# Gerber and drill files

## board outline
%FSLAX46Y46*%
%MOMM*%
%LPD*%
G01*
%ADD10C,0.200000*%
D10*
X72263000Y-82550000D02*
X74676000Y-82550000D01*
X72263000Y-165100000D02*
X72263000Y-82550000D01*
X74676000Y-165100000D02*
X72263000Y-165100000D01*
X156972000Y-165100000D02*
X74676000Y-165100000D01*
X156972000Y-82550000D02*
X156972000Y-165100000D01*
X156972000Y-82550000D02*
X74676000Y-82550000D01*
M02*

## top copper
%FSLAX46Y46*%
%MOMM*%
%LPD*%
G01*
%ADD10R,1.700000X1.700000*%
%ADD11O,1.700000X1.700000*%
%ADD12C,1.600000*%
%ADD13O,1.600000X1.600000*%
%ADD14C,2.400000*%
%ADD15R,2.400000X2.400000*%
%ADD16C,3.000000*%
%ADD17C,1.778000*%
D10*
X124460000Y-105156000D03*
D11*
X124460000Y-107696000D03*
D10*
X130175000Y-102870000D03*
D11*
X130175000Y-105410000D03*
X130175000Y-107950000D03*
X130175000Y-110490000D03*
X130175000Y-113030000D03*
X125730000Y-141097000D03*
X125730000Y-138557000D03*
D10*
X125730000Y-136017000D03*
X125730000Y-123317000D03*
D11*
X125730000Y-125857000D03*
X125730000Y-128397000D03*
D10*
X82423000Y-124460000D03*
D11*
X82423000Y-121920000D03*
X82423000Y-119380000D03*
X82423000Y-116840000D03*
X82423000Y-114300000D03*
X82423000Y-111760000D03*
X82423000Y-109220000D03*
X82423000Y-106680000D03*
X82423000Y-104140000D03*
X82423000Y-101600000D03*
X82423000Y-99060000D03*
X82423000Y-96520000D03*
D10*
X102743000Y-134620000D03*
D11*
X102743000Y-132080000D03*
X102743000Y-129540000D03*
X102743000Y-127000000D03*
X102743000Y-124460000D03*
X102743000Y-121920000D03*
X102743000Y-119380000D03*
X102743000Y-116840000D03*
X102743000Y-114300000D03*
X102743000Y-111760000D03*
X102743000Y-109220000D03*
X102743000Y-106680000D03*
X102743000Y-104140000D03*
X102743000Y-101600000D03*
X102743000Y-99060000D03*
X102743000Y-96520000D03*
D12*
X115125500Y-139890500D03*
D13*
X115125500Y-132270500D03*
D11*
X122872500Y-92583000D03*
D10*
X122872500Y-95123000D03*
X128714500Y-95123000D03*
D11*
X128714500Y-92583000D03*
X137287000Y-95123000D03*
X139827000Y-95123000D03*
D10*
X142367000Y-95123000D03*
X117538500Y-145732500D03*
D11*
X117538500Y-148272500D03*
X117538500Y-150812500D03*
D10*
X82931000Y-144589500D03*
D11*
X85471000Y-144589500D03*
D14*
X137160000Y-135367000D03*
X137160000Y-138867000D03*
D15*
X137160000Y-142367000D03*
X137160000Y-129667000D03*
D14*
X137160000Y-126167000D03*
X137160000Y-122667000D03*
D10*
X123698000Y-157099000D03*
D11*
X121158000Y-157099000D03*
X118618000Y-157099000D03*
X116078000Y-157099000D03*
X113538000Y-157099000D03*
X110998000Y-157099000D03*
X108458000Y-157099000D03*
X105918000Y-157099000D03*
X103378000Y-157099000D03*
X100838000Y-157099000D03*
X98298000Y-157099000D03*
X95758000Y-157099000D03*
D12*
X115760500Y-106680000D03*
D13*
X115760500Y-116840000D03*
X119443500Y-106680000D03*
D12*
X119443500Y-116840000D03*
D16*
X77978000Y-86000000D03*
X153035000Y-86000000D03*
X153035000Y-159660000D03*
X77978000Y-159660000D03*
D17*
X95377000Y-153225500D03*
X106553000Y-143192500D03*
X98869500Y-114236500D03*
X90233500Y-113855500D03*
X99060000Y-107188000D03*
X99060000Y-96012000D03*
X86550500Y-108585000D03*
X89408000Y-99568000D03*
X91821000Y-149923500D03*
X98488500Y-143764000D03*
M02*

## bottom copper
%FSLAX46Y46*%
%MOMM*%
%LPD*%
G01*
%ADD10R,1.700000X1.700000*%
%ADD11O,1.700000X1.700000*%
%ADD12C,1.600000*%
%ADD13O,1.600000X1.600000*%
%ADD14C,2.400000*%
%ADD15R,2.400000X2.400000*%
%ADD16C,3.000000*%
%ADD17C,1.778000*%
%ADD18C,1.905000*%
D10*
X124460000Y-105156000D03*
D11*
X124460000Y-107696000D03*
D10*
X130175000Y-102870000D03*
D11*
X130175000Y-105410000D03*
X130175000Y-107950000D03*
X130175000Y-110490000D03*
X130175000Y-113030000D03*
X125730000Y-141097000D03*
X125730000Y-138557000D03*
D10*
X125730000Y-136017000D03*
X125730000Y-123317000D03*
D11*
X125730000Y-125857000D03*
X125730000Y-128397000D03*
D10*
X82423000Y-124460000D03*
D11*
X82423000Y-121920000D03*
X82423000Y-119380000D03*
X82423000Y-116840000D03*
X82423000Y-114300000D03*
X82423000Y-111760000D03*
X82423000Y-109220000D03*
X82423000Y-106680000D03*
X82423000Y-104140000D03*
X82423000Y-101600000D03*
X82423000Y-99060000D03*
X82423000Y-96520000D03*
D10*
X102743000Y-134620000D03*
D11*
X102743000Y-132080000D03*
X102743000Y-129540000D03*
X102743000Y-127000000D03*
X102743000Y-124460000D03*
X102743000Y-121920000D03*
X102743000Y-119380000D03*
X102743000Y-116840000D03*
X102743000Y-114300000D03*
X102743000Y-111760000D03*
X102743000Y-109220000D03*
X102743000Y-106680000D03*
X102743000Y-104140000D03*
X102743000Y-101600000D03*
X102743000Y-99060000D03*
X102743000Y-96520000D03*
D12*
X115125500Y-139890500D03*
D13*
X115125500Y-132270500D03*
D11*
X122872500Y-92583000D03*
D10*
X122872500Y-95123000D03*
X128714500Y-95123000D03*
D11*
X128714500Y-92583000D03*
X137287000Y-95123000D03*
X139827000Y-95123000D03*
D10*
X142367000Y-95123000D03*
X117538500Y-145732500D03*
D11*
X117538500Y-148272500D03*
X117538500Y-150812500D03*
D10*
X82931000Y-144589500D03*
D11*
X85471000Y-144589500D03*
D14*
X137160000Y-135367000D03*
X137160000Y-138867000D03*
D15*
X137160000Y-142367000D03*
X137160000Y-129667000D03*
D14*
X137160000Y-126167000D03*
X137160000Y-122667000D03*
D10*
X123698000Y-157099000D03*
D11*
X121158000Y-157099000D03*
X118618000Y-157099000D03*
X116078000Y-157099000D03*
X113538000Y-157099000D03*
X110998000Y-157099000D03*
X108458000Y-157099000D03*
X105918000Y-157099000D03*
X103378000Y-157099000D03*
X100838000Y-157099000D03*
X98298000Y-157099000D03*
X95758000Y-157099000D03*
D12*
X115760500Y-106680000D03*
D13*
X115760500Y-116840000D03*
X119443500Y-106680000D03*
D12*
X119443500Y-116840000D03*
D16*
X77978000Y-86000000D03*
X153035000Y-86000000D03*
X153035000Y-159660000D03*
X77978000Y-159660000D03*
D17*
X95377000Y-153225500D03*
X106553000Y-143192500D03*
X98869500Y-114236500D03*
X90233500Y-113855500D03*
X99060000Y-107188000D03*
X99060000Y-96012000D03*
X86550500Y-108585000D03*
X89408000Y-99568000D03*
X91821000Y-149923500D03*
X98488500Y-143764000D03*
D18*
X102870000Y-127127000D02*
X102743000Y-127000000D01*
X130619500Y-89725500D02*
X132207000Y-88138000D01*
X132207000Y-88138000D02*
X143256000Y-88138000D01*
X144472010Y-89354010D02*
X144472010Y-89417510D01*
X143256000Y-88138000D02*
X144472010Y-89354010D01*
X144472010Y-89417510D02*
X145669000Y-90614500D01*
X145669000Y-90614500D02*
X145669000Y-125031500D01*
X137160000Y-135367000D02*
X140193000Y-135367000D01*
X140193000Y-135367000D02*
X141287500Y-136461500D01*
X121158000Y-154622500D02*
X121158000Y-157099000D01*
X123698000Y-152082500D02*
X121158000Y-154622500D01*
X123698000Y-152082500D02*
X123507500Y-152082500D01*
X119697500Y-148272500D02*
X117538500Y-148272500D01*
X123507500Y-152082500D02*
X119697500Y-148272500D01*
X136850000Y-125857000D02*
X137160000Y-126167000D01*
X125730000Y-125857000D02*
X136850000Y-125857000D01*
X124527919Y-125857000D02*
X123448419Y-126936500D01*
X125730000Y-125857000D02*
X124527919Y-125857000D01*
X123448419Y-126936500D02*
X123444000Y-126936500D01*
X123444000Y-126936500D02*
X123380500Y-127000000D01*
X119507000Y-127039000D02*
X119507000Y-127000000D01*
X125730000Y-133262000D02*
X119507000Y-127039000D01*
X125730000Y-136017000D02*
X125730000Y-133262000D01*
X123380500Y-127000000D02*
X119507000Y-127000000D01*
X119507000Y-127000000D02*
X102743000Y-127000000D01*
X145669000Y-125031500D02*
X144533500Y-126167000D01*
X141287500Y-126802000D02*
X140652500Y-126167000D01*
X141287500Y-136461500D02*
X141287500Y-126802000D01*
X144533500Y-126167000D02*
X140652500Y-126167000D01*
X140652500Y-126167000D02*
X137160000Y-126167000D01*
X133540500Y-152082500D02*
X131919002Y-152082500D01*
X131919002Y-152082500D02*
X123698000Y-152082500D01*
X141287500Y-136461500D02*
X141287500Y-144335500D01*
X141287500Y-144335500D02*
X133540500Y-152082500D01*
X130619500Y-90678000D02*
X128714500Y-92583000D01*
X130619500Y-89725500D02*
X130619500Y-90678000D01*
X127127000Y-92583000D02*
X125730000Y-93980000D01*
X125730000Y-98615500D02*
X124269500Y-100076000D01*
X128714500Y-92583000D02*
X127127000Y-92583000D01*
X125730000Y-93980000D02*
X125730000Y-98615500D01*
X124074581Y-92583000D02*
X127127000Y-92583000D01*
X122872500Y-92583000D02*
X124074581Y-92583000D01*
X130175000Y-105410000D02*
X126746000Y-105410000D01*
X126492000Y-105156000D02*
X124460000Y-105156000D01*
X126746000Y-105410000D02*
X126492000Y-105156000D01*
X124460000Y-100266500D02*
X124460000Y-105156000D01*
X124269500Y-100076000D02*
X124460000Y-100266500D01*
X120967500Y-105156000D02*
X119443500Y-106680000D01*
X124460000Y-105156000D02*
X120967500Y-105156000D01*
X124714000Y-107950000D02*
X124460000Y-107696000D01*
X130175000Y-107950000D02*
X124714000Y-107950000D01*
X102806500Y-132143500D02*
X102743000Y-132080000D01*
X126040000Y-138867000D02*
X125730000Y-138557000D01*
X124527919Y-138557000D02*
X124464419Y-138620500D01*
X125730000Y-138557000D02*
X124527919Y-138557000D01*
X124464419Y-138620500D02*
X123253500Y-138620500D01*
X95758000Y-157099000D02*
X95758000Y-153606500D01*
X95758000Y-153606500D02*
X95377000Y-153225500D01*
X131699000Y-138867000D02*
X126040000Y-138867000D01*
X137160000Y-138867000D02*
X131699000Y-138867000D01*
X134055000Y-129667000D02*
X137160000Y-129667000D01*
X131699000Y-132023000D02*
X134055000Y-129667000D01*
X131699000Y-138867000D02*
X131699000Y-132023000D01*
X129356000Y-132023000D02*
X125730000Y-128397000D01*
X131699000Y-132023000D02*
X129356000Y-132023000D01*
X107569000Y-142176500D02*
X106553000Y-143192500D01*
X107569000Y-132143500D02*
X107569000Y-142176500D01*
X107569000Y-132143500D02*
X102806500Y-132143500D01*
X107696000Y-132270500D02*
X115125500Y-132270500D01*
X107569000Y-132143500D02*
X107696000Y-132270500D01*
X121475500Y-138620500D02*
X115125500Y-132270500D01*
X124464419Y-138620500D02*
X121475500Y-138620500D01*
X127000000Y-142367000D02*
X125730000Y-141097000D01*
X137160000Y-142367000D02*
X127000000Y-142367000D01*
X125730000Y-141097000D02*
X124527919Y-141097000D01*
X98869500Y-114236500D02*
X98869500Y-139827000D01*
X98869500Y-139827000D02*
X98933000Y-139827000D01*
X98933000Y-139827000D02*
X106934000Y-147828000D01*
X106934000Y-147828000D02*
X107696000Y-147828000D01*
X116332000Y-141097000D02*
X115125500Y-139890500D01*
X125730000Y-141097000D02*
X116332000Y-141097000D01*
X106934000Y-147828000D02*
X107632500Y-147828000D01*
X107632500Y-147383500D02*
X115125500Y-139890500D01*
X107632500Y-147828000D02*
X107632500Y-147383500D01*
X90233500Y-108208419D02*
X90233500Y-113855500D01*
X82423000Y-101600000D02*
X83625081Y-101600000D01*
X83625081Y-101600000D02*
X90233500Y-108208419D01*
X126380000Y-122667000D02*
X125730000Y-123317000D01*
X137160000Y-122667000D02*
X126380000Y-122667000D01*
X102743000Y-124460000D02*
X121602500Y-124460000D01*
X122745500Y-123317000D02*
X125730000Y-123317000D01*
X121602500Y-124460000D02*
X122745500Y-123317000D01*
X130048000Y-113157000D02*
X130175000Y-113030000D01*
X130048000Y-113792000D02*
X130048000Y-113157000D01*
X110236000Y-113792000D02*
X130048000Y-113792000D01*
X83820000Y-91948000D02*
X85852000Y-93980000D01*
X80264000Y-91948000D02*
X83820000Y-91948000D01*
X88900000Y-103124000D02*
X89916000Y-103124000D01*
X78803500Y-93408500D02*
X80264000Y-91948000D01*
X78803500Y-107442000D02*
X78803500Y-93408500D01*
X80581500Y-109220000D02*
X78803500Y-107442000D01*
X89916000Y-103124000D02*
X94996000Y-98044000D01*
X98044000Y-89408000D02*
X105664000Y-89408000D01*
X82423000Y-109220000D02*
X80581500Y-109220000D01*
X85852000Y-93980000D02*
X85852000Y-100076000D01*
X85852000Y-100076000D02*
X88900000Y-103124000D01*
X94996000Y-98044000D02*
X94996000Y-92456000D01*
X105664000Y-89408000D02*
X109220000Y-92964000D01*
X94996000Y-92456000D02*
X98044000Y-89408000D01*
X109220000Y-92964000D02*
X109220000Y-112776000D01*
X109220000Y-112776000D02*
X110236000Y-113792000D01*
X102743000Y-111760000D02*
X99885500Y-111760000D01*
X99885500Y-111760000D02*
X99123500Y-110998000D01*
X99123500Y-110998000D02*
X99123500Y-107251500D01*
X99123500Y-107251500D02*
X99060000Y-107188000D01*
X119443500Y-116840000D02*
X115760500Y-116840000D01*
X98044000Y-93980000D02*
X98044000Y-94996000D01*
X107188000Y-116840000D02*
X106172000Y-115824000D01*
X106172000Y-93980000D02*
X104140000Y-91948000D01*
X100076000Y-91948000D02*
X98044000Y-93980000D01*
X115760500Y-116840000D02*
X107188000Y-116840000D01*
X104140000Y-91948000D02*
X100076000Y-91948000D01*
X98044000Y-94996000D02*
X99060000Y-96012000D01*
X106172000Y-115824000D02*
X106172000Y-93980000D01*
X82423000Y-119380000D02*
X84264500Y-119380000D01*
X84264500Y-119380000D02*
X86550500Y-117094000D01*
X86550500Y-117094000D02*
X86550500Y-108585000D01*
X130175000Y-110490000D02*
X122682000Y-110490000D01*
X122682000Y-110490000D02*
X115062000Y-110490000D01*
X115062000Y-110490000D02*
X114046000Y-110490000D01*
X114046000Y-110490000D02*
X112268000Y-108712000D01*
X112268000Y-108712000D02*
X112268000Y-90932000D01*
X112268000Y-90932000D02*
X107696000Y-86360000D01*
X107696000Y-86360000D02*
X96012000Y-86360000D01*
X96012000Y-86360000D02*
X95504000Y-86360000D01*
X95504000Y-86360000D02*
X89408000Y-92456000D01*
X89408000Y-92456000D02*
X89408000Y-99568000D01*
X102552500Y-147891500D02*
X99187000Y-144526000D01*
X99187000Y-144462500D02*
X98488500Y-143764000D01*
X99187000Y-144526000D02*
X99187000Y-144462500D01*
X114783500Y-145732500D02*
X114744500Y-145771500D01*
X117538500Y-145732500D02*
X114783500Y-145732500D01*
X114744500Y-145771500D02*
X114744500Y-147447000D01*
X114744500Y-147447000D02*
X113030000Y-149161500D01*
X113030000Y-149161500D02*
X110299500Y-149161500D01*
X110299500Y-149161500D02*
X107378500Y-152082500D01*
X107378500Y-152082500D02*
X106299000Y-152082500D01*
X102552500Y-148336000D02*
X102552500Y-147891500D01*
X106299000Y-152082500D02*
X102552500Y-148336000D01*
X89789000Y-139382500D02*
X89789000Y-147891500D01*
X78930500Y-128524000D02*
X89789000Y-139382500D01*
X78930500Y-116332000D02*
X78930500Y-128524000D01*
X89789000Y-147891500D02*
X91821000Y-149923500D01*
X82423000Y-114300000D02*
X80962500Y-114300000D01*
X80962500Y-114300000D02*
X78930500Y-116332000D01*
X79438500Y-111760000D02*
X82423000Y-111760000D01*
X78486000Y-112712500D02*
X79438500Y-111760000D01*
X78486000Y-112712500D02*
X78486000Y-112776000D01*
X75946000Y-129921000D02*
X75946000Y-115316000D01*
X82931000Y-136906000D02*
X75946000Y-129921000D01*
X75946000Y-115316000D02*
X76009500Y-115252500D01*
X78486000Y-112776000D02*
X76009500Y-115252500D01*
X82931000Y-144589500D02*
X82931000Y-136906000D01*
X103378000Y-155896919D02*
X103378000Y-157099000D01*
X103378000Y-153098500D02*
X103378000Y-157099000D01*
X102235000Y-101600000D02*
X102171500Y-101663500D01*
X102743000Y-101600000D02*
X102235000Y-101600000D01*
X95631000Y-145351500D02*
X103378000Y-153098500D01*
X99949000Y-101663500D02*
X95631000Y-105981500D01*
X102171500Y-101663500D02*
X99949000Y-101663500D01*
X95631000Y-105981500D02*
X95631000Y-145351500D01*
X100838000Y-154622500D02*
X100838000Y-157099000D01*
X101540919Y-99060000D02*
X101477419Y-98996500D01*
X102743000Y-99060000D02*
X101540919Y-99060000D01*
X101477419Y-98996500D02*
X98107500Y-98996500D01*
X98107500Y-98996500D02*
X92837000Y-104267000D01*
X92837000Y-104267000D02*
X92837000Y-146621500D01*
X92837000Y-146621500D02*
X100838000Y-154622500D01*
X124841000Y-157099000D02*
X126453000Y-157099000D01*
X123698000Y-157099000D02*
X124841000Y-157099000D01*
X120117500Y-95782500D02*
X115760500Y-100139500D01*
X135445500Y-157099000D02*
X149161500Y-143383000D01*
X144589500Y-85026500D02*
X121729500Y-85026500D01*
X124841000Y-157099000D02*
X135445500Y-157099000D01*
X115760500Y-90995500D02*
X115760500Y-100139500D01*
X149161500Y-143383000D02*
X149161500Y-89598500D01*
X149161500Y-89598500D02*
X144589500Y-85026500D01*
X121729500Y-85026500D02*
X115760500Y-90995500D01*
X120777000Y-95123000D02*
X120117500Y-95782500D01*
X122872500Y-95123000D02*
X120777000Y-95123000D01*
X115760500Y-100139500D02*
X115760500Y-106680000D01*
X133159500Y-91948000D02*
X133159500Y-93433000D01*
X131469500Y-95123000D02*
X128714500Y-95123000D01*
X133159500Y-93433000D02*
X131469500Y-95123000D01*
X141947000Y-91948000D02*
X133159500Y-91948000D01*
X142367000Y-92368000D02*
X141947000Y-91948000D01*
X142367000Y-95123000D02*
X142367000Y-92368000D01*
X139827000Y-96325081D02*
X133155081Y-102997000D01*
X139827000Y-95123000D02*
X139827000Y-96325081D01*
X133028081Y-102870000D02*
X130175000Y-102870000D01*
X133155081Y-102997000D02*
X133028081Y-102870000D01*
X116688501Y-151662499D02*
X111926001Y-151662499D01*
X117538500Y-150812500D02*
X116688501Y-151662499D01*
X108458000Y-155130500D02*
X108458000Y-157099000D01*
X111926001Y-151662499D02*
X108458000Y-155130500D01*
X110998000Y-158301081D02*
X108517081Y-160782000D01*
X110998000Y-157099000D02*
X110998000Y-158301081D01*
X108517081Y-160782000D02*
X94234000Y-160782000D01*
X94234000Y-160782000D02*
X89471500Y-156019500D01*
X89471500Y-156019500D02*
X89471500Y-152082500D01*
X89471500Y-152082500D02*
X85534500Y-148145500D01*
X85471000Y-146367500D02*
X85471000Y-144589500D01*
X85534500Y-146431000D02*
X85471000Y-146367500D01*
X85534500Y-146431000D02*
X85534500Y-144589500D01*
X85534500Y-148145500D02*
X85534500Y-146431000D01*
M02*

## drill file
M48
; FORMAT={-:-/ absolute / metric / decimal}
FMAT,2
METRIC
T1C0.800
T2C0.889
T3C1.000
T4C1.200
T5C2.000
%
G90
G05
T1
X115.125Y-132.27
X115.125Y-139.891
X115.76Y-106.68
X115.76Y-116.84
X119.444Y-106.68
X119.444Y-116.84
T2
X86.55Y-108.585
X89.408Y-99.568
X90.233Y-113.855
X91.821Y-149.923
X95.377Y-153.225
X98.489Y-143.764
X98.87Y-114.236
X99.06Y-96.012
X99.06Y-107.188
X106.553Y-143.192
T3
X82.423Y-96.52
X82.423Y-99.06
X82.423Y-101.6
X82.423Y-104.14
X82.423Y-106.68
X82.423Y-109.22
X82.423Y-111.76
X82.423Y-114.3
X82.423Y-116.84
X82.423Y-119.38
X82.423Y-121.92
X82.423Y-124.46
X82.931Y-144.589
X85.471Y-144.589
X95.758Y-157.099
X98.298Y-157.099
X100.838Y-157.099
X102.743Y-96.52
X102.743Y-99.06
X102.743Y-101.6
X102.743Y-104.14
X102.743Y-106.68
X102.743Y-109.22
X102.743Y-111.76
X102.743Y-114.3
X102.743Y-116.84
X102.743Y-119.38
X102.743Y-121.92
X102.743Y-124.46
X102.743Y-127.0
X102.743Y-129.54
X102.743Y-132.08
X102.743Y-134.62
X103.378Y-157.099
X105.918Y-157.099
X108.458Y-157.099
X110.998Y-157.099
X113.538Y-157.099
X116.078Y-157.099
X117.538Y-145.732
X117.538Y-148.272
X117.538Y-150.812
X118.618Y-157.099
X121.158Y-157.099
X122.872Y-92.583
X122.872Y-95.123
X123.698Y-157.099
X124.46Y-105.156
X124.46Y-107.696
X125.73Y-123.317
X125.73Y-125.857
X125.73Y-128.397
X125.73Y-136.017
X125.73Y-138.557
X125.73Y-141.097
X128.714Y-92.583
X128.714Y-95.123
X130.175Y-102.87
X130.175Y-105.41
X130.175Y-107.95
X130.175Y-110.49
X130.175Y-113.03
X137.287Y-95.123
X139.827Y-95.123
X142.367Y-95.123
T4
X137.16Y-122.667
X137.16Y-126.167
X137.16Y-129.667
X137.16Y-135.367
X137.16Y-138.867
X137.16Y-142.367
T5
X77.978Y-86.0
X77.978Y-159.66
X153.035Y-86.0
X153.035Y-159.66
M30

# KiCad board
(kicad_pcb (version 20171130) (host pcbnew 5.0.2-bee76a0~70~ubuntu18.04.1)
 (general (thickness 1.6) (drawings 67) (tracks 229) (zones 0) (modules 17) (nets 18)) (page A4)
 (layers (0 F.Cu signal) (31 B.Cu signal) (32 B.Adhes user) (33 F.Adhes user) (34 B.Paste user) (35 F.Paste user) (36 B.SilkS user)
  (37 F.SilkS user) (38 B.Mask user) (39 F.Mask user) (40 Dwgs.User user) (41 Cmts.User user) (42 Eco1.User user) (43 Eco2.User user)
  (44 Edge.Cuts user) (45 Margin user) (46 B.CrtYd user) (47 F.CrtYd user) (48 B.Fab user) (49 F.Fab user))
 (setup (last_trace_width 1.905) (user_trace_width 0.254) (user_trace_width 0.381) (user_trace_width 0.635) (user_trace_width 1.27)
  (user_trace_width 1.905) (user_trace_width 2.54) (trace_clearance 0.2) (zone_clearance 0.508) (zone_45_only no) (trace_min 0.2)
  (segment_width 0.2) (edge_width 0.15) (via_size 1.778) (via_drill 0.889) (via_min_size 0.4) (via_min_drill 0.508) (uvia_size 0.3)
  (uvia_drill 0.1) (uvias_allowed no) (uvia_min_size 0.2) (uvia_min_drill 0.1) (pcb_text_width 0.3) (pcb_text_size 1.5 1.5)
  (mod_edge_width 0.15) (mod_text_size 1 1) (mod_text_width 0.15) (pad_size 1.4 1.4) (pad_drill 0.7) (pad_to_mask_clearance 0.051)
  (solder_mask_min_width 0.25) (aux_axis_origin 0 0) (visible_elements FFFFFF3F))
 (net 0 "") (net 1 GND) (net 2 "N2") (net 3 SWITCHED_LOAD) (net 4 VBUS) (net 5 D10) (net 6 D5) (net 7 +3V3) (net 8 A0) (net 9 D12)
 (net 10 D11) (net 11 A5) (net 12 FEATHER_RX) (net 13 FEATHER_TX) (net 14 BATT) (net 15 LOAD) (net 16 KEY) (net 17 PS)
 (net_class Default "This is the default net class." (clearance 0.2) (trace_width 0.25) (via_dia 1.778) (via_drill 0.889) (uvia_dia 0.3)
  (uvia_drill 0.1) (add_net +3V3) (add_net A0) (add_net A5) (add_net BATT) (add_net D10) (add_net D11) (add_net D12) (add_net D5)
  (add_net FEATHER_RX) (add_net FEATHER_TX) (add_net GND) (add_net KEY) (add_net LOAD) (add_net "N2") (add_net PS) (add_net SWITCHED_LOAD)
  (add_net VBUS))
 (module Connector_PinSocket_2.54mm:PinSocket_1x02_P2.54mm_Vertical (layer F.Cu) (at 124.46 105.156)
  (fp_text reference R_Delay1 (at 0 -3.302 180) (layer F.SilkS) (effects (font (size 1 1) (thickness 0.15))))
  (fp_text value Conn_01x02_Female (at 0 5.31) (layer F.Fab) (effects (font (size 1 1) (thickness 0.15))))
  (pad 1 thru_hole rect (at 0 0) (size 1.7 1.7) (drill 1) (layers *.Cu *.Mask) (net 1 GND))
  (pad 2 thru_hole oval (at 0 2.54) (size 1.7 1.7) (drill 1) (layers *.Cu *.Mask) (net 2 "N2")))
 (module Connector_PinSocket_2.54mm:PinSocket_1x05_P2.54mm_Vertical (layer F.Cu) (at 130.175 102.87)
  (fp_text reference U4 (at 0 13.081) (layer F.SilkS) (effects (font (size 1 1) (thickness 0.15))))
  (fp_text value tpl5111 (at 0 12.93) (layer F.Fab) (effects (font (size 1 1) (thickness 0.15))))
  (pad 1 thru_hole rect (at 0 0) (size 1.7 1.7) (drill 1) (layers *.Cu *.Mask) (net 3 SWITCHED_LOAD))
  (pad 2 thru_hole oval (at 0 2.54) (size 1.7 1.7) (drill 1) (layers *.Cu *.Mask) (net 1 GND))
  (pad 3 thru_hole oval (at 0 5.08) (size 1.7 1.7) (drill 1) (layers *.Cu *.Mask) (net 2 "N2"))
  (pad 4 thru_hole oval (at 0 7.62) (size 1.7 1.7) (drill 1) (layers *.Cu *.Mask) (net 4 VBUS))
  (pad 5 thru_hole oval (at 0 10.16) (size 1.7 1.7) (drill 1) (layers *.Cu *.Mask) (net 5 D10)))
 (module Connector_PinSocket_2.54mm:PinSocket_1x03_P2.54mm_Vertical (layer F.Cu) (at 125.73 136.017)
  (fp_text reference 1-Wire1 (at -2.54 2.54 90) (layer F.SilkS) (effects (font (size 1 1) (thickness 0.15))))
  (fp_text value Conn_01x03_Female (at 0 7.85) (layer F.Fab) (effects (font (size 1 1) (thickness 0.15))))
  (pad 3 thru_hole oval (at 0 5.08) (size 1.7 1.7) (drill 1) (layers *.Cu *.Mask) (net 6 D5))
  (pad 2 thru_hole oval (at 0 2.54) (size 1.7 1.7) (drill 1) (layers *.Cu *.Mask) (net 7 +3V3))
  (pad 1 thru_hole rect (at 0 0) (size 1.7 1.7) (drill 1) (layers *.Cu *.Mask) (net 1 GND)))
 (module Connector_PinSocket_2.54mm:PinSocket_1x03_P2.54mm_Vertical (layer F.Cu) (at 125.73 123.317)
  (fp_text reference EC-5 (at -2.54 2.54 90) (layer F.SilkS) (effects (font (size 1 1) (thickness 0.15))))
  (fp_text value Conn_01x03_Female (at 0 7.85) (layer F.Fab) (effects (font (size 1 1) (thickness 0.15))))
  (pad 1 thru_hole rect (at 0 0) (size 1.7 1.7) (drill 1) (layers *.Cu *.Mask) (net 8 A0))
  (pad 2 thru_hole oval (at 0 2.54) (size 1.7 1.7) (drill 1) (layers *.Cu *.Mask) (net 1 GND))
  (pad 3 thru_hole oval (at 0 5.08) (size 1.7 1.7) (drill 1) (layers *.Cu *.Mask) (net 7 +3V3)))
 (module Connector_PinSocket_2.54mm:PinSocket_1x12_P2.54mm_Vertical (layer F.Cu) (at 82.423 124.46 180)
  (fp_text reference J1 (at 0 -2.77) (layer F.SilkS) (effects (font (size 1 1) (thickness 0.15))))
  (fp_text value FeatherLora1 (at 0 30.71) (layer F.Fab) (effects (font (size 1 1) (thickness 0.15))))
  (pad 1 thru_hole rect (at 0 0 180) (size 1.7 1.7) (drill 1) (layers *.Cu *.Mask))
  (pad 2 thru_hole oval (at 0 2.54 180) (size 1.7 1.7) (drill 1) (layers *.Cu *.Mask))
  (pad 3 thru_hole oval (at 0 5.08 180) (size 1.7 1.7) (drill 1) (layers *.Cu *.Mask) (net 4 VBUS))
  (pad 4 thru_hole oval (at 0 7.62 180) (size 1.7 1.7) (drill 1) (layers *.Cu *.Mask))
  (pad 5 thru_hole oval (at 0 10.16 180) (size 1.7 1.7) (drill 1) (layers *.Cu *.Mask) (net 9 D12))
  (pad 6 thru_hole oval (at 0 12.7 180) (size 1.7 1.7) (drill 1) (layers *.Cu *.Mask) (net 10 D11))
  (pad 7 thru_hole oval (at 0 15.24 180) (size 1.7 1.7) (drill 1) (layers *.Cu *.Mask) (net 5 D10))
  (pad 8 thru_hole oval (at 0 17.78 180) (size 1.7 1.7) (drill 1) (layers *.Cu *.Mask))
  (pad 9 thru_hole oval (at 0 20.32 180) (size 1.7 1.7) (drill 1) (layers *.Cu *.Mask))
  (pad 10 thru_hole oval (at 0 22.86 180) (size 1.7 1.7) (drill 1) (layers *.Cu *.Mask) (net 6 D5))
  (pad 11 thru_hole oval (at 0 25.4 180) (size 1.7 1.7) (drill 1) (layers *.Cu *.Mask))
  (pad 12 thru_hole oval (at 0 27.94 180) (size 1.7 1.7) (drill 1) (layers *.Cu *.Mask)))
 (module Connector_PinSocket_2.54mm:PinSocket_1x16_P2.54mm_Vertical (layer F.Cu) (at 102.743 134.62 180)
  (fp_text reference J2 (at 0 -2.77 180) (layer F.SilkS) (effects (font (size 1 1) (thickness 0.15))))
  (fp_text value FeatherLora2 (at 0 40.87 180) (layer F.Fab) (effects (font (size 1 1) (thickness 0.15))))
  (pad 1 thru_hole rect (at 0 0 180) (size 1.7 1.7) (drill 1) (layers *.Cu *.Mask))
  (pad 2 thru_hole oval (at 0 2.54 180) (size 1.7 1.7) (drill 1) (layers *.Cu *.Mask) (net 7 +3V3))
  (pad 3 thru_hole oval (at 0 5.08 180) (size 1.7 1.7) (drill 1) (layers *.Cu *.Mask))
  (pad 4 thru_hole oval (at 0 7.62 180) (size 1.7 1.7) (drill 1) (layers *.Cu *.Mask) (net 1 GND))
  (pad 5 thru_hole oval (at 0 10.16 180) (size 1.7 1.7) (drill 1) (layers *.Cu *.Mask) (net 8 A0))
  (pad 6 thru_hole oval (at 0 12.7 180) (size 1.7 1.7) (drill 1) (layers *.Cu *.Mask))
  (pad 7 thru_hole oval (at 0 15.24 180) (size 1.7 1.7) (drill 1) (layers *.Cu *.Mask))
  (pad 8 thru_hole oval (at 0 17.78 180) (size 1.7 1.7) (drill 1) (layers *.Cu *.Mask))
  (pad 9 thru_hole oval (at 0 20.32 180) (size 1.7 1.7) (drill 1) (layers *.Cu *.Mask))
  (pad 10 thru_hole oval (at 0 22.86 180) (size 1.7 1.7) (drill 1) (layers *.Cu *.Mask) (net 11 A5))
  (pad 11 thru_hole oval (at 0 25.4 180) (size 1.7 1.7) (drill 1) (layers *.Cu *.Mask))
  (pad 12 thru_hole oval (at 0 27.94 180) (size 1.7 1.7) (drill 1) (layers *.Cu *.Mask))
  (pad 13 thru_hole oval (at 0 30.48 180) (size 1.7 1.7) (drill 1) (layers *.Cu *.Mask))
  (pad 14 thru_hole oval (at 0 33.02 180) (size 1.7 1.7) (drill 1) (layers *.Cu *.Mask) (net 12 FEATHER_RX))
  (pad 15 thru_hole oval (at 0 35.56 180) (size 1.7 1.7) (drill 1) (layers *.Cu *.Mask) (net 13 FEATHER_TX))
  (pad 16 thru_hole oval (at 0 38.1 180) (size 1.7 1.7) (drill 1) (layers *.Cu *.Mask)))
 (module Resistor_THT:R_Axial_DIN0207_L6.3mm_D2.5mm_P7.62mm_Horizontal (layer F.Cu) (at 115.1255 139.8905 90)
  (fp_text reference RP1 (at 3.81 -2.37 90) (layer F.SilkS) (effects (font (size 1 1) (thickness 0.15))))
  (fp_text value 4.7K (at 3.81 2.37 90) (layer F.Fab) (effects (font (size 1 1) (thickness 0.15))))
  (pad 1 thru_hole circle (at 0 0 90) (size 1.6 1.6) (drill 0.8) (layers *.Cu *.Mask) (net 6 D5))
  (pad 2 thru_hole oval (at 7.62 0 90) (size 1.6 1.6) (drill 0.8) (layers *.Cu *.Mask) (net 7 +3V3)))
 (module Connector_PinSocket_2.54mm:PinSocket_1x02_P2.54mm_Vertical (layer F.Cu) (at 122.8725 95.123 180)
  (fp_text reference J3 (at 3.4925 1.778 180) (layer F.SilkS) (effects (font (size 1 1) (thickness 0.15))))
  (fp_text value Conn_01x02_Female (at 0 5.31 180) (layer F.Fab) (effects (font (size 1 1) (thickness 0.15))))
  (pad 2 thru_hole oval (at 0 2.54 180) (size 1.7 1.7) (drill 1) (layers *.Cu *.Mask) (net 1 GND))
  (pad 1 thru_hole rect (at 0 0 180) (size 1.7 1.7) (drill 1) (layers *.Cu *.Mask) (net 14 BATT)))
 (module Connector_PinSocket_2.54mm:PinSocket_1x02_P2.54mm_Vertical (layer F.Cu) (at 128.7145 95.123 180)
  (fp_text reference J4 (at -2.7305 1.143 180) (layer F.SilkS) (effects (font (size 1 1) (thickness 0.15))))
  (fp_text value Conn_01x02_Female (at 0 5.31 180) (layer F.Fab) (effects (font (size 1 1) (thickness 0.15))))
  (pad 1 thru_hole rect (at 0 0 180) (size 1.7 1.7) (drill 1) (layers *.Cu *.Mask) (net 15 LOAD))
  (pad 2 thru_hole oval (at 0 2.54 180) (size 1.7 1.7) (drill 1) (layers *.Cu *.Mask) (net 1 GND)))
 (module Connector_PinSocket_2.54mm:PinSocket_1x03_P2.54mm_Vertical (layer F.Cu) (at 142.367 95.123 270)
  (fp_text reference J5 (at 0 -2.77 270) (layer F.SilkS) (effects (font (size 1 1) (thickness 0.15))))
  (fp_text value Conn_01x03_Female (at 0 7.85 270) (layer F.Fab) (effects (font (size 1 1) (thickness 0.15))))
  (pad 3 thru_hole oval (at 0 5.08 270) (size 1.7 1.7) (drill 1) (layers *.Cu *.Mask))
  (pad 2 thru_hole oval (at 0 2.54 270) (size 1.7 1.7) (drill 1) (layers *.Cu *.Mask) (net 3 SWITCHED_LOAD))
  (pad 1 thru_hole rect (at 0 0 270) (size 1.7 1.7) (drill 1) (layers *.Cu *.Mask) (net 15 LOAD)))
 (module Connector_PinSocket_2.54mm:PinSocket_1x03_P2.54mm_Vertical (layer F.Cu) (at 117.5385 145.7325)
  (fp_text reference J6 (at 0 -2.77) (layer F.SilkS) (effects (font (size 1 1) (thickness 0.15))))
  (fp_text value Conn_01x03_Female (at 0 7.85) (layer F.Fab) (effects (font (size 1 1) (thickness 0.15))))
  (pad 1 thru_hole rect (at 0 0) (size 1.7 1.7) (drill 1) (layers *.Cu *.Mask) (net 9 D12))
  (pad 2 thru_hole oval (at 0 2.54) (size 1.7 1.7) (drill 1) (layers *.Cu *.Mask) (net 1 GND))
  (pad 3 thru_hole oval (at 0 5.08) (size 1.7 1.7) (drill 1) (layers *.Cu *.Mask) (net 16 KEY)))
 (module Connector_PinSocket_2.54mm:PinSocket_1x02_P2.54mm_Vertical (layer F.Cu) (at 82.931 144.5895 90)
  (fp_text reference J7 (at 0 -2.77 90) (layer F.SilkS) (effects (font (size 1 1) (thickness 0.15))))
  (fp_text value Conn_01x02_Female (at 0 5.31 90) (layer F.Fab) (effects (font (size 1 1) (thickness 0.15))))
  (pad 1 thru_hole rect (at 0 0 90) (size 1.7 1.7) (drill 1) (layers *.Cu *.Mask) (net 10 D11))
  (pad 2 thru_hole oval (at 0 2.54 90) (size 1.7 1.7) (drill 1) (layers *.Cu *.Mask) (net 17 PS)))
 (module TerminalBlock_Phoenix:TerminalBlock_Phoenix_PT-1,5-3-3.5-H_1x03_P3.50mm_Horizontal (layer F.Cu) (at 137.16 142.367 90)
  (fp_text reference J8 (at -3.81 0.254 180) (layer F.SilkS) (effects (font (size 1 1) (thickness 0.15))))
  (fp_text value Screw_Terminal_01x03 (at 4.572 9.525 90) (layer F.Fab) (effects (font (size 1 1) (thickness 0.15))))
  (pad 3 thru_hole circle (at 7 0 90) (size 2.4 2.4) (drill 1.2) (layers *.Cu *.Mask) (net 1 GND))
  (pad 2 thru_hole circle (at 3.5 0 90) (size 2.4 2.4) (drill 1.2) (layers *.Cu *.Mask) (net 7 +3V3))
  (pad 1 thru_hole rect (at 0 0 90) (size 2.4 2.4) (drill 1.2) (layers *.Cu *.Mask) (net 6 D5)))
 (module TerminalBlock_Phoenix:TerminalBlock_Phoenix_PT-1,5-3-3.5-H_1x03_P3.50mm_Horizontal (layer F.Cu) (at 137.16 129.667 90)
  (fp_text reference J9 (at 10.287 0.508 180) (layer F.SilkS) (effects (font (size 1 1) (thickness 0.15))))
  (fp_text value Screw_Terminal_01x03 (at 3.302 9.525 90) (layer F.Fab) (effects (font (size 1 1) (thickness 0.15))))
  (pad 1 thru_hole rect (at 0 0 90) (size 2.4 2.4) (drill 1.2) (layers *.Cu *.Mask) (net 7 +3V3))
  (pad 2 thru_hole circle (at 3.5 0 90) (size 2.4 2.4) (drill 1.2) (layers *.Cu *.Mask) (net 1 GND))
  (pad 3 thru_hole circle (at 7 0 90) (size 2.4 2.4) (drill 1.2) (layers *.Cu *.Mask) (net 8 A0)))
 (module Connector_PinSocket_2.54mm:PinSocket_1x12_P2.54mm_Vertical (layer F.Cu) (at 123.698 157.099 270)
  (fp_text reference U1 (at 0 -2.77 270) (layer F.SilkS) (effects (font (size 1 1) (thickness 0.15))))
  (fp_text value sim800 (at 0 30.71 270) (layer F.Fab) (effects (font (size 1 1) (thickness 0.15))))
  (pad 1 thru_hole rect (at 0 0 270) (size 1.7 1.7) (drill 1) (layers *.Cu *.Mask) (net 14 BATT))
  (pad 2 thru_hole oval (at 0 2.54 270) (size 1.7 1.7) (drill 1) (layers *.Cu *.Mask) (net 1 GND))
  (pad 3 thru_hole oval (at 0 5.08 270) (size 1.7 1.7) (drill 1) (layers *.Cu *.Mask))
  (pad 4 thru_hole oval (at 0 7.62 270) (size 1.7 1.7) (drill 1) (layers *.Cu *.Mask))
  (pad 5 thru_hole oval (at 0 10.16 270) (size 1.7 1.7) (drill 1) (layers *.Cu *.Mask))
  (pad 6 thru_hole oval (at 0 12.7 270) (size 1.7 1.7) (drill 1) (layers *.Cu *.Mask) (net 17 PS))
  (pad 7 thru_hole oval (at 0 15.24 270) (size 1.7 1.7) (drill 1) (layers *.Cu *.Mask) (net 16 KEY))
  (pad 8 thru_hole oval (at 0 17.78 270) (size 1.7 1.7) (drill 1) (layers *.Cu *.Mask))
  (pad 9 thru_hole oval (at 0 20.32 270) (size 1.7 1.7) (drill 1) (layers *.Cu *.Mask) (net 12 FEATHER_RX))
  (pad 10 thru_hole oval (at 0 22.86 270) (size 1.7 1.7) (drill 1) (layers *.Cu *.Mask) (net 13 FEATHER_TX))
  (pad 11 thru_hole oval (at 0 25.4 270) (size 1.7 1.7) (drill 1) (layers *.Cu *.Mask))
  (pad 12 thru_hole oval (at 0 27.94 270) (size 1.7 1.7) (drill 1) (layers *.Cu *.Mask) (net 7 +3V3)))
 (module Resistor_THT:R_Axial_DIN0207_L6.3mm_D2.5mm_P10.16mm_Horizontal (layer F.Cu) (at 115.7605 106.68 270)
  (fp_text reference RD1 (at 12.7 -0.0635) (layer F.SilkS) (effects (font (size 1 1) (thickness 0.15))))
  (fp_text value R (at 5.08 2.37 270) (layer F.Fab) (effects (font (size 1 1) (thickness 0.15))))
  (pad 1 thru_hole circle (at 0 0 270) (size 1.6 1.6) (drill 0.8) (layers *.Cu *.Mask) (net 14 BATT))
  (pad 2 thru_hole oval (at 10.16 0 270) (size 1.6 1.6) (drill 0.8) (layers *.Cu *.Mask) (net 11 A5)))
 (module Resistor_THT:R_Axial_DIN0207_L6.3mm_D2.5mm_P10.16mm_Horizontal (layer F.Cu) (at 119.4435 116.84 90)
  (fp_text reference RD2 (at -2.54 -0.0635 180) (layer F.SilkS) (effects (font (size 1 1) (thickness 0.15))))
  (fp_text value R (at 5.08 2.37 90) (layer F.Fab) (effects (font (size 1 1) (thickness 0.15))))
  (pad 2 thru_hole oval (at 10.16 0 90) (size 1.6 1.6) (drill 0.8) (layers *.Cu *.Mask) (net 1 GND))
  (pad 1 thru_hole circle (at 0 0 90) (size 1.6 1.6) (drill 0.8) (layers *.Cu *.Mask) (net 11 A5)))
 (gr_line (start 72.263 82.55) (end 74.676 82.55) (layer Edge.Cuts) (width 0.2))
 (gr_line (start 72.263 165.1) (end 72.263 82.55) (layer Edge.Cuts) (width 0.2))
 (gr_line (start 74.676 165.1) (end 72.263 165.1) (layer Edge.Cuts) (width 0.2))
 (gr_line (start 156.972 165.1) (end 74.676 165.1) (layer Edge.Cuts) (width 0.2))
 (gr_line (start 156.972 82.55) (end 156.972 165.1) (layer Edge.Cuts) (width 0.2))
 (gr_line (start 156.972 82.55) (end 74.676 82.55) (layer Edge.Cuts) (width 0.2))
 (via (at 77.978 86) (size 3) (drill 2) (layers F.Cu B.Cu) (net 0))
 (via (at 153.035 86) (size 3) (drill 2) (layers F.Cu B.Cu) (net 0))
 (via (at 153.035 159.66) (size 3) (drill 2) (layers F.Cu B.Cu) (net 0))
 (via (at 77.978 159.66) (size 3) (drill 2) (layers F.Cu B.Cu) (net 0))
 (segment (start 102.87 127.127) (end 102.743 127) (width 1.905) (layer B.Cu) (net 1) (status 30))
 (segment (start 130.6195 89.7255) (end 132.207 88.138) (width 1.905) (layer B.Cu) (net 1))
 (segment (start 132.207 88.138) (end 143.256 88.138) (width 1.905) (layer B.Cu) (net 1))
 (segment (start 144.47201 89.35401) (end 144.47201 89.41751) (width 1.905) (layer B.Cu) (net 1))
 (segment (start 143.256 88.138) (end 144.47201 89.35401) (width 1.905) (layer B.Cu) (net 1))
 (segment (start 144.47201 89.41751) (end 145.669 90.6145) (width 1.905) (layer B.Cu) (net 1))
 (segment (start 145.669 90.6145) (end 145.669 125.0315) (width 1.905) (layer B.Cu) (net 1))
 (segment (start 137.16 135.367) (end 140.193 135.367) (width 1.905) (layer B.Cu) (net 1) (status 10))
 (segment (start 140.193 135.367) (end 141.2875 136.4615) (width 1.905) (layer B.Cu) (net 1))
 (segment (start 121.158 154.6225) (end 121.158 157.099) (width 1.905) (layer B.Cu) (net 1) (status 20))
 (segment (start 123.698 152.0825) (end 121.158 154.6225) (width 1.905) (layer B.Cu) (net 1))
 (segment (start 123.698 152.0825) (end 123.5075 152.0825) (width 1.905) (layer B.Cu) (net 1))
 (segment (start 119.6975 148.2725) (end 117.5385 148.2725) (width 1.905) (layer B.Cu) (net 1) (status 20))
 (segment (start 123.5075 152.0825) (end 119.6975 148.2725) (width 1.905) (layer B.Cu) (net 1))
 (segment (start 136.85 125.857) (end 137.16 126.167) (width 1.905) (layer B.Cu) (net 1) (status 30))
 (segment (start 125.73 125.857) (end 136.85 125.857) (width 1.905) (layer B.Cu) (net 1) (status 30))
 (segment (start 124.527919 125.857) (end 123.448419 126.9365) (width 1.905) (layer B.Cu) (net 1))
 (segment (start 125.73 125.857) (end 124.527919 125.857) (width 1.905) (layer B.Cu) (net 1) (status 10))
 (segment (start 123.448419 126.9365) (end 123.444 126.9365) (width 1.905) (layer B.Cu) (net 1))
 (segment (start 123.444 126.9365) (end 123.3805 127) (width 1.905) (layer B.Cu) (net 1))
 (segment (start 119.507 127.039) (end 119.507 127) (width 1.905) (layer B.Cu) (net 1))
 (segment (start 125.73 133.262) (end 119.507 127.039) (width 1.905) (layer B.Cu) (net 1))
 (segment (start 125.73 136.017) (end 125.73 133.262) (width 1.905) (layer B.Cu) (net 1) (status 10))
 (segment (start 123.3805 127) (end 119.507 127) (width 1.905) (layer B.Cu) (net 1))
 (segment (start 119.507 127) (end 102.743 127) (width 1.905) (layer B.Cu) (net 1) (status 20))
 (segment (start 145.669 125.0315) (end 144.5335 126.167) (width 1.905) (layer B.Cu) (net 1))
 (segment (start 141.2875 126.802) (end 140.6525 126.167) (width 1.905) (layer B.Cu) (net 1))
 (segment (start 141.2875 136.4615) (end 141.2875 126.802) (width 1.905) (layer B.Cu) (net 1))
 (segment (start 144.5335 126.167) (end 140.6525 126.167) (width 1.905) (layer B.Cu) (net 1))
 (segment (start 140.6525 126.167) (end 137.16 126.167) (width 1.905) (layer B.Cu) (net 1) (status 20))
 (segment (start 133.5405 152.0825) (end 131.919002 152.0825) (width 1.905) (layer B.Cu) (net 1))
 (segment (start 131.919002 152.0825) (end 123.698 152.0825) (width 1.905) (layer B.Cu) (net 1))
 (segment (start 141.2875 136.4615) (end 141.2875 144.3355) (width 1.905) (layer B.Cu) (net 1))
 (segment (start 141.2875 144.3355) (end 133.5405 152.0825) (width 1.905) (layer B.Cu) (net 1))
 (segment (start 130.6195 90.678) (end 128.7145 92.583) (width 1.905) (layer B.Cu) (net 1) (status 20))
 (segment (start 130.6195 89.7255) (end 130.6195 90.678) (width 1.905) (layer B.Cu) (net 1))
 (segment (start 127.127 92.583) (end 125.73 93.98) (width 1.905) (layer B.Cu) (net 1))
 (segment (start 125.73 98.6155) (end 124.2695 100.076) (width 1.905) (layer B.Cu) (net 1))
 (segment (start 128.7145 92.583) (end 127.127 92.583) (width 1.905) (layer B.Cu) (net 1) (status 10))
 (segment (start 125.73 93.98) (end 125.73 98.6155) (width 1.905) (layer B.Cu) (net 1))
 (segment (start 124.074581 92.583) (end 127.127 92.583) (width 1.905) (layer B.Cu) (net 1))
 (segment (start 122.8725 92.583) (end 124.074581 92.583) (width 1.905) (layer B.Cu) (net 1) (status 10))
 (segment (start 130.175 105.41) (end 126.746 105.41) (width 1.905) (layer B.Cu) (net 1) (status 10))
 (segment (start 126.492 105.156) (end 124.46 105.156) (width 1.905) (layer B.Cu) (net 1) (status 20))
 (segment (start 126.746 105.41) (end 126.492 105.156) (width 1.905) (layer B.Cu) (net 1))
 (segment (start 124.46 100.2665) (end 124.46 105.156) (width 1.905) (layer B.Cu) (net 1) (status 20))
 (segment (start 124.2695 100.076) (end 124.46 100.2665) (width 1.905) (layer B.Cu) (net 1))
 (segment (start 120.9675 105.156) (end 119.4435 106.68) (width 1.905) (layer B.Cu) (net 1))
 (segment (start 124.46 105.156) (end 120.9675 105.156) (width 1.905) (layer B.Cu) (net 1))
 (segment (start 124.714 107.95) (end 124.46 107.696) (width 1.905) (layer B.Cu) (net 2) (status 30))
 (segment (start 130.175 107.95) (end 124.714 107.95) (width 1.905) (layer B.Cu) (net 2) (status 30))
 (segment (start 102.8065 132.1435) (end 102.743 132.08) (width 1.905) (layer B.Cu) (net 7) (status 30))
 (segment (start 126.04 138.867) (end 125.73 138.557) (width 1.905) (layer B.Cu) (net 7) (status 30))
 (segment (start 124.527919 138.557) (end 124.464419 138.6205) (width 1.905) (layer B.Cu) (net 7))
 (segment (start 125.73 138.557) (end 124.527919 138.557) (width 1.905) (layer B.Cu) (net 7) (status 10))
 (segment (start 124.464419 138.6205) (end 123.2535 138.6205) (width 1.905) (layer B.Cu) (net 7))
 (segment (start 95.758 157.099) (end 95.758 153.6065) (width 1.905) (layer B.Cu) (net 7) (status 10))
 (via (at 95.377 153.2255) (size 1.778) (drill 0.889) (layers F.Cu B.Cu) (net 7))
 (segment (start 95.758 153.6065) (end 95.377 153.2255) (width 1.905) (layer B.Cu) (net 7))
 (segment (start 131.699 138.867) (end 126.04 138.867) (width 1.905) (layer B.Cu) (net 7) (status 20))
 (segment (start 137.16 138.867) (end 131.699 138.867) (width 1.905) (layer B.Cu) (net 7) (status 10))
 (segment (start 134.055 129.667) (end 137.16 129.667) (width 1.905) (layer B.Cu) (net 7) (status 20))
 (segment (start 131.699 132.023) (end 134.055 129.667) (width 1.905) (layer B.Cu) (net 7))
 (segment (start 131.699 138.867) (end 131.699 132.023) (width 1.905) (layer B.Cu) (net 7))
 (segment (start 129.356 132.023) (end 125.73 128.397) (width 1.905) (layer B.Cu) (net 7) (status 20))
 (segment (start 131.699 132.023) (end 129.356 132.023) (width 1.905) (layer B.Cu) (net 7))
 (via (at 106.553 143.1925) (size 1.778) (drill 0.889) (layers F.Cu B.Cu) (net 7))
 (segment (start 107.569 142.1765) (end 106.553 143.1925) (width 1.905) (layer B.Cu) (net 7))
 (segment (start 107.569 132.1435) (end 107.569 142.1765) (width 1.905) (layer B.Cu) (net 7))
 (segment (start 107.569 132.1435) (end 102.8065 132.1435) (width 1.905) (layer B.Cu) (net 7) (status 20))
 (segment (start 107.696 132.2705) (end 115.1255 132.2705) (width 1.905) (layer B.Cu) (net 7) (status 20))
 (segment (start 107.569 132.1435) (end 107.696 132.2705) (width 1.905) (layer B.Cu) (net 7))
 (segment (start 121.4755 138.6205) (end 115.1255 132.2705) (width 1.905) (layer B.Cu) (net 7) (status 20))
 (segment (start 124.464419 138.6205) (end 121.4755 138.6205) (width 1.905) (layer B.Cu) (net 7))
 (via (at 98.8695 114.2365) (size 1.778) (drill 0.889) (layers F.Cu B.Cu) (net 6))
 (segment (start 127 142.367) (end 125.73 141.097) (width 1.905) (layer B.Cu) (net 6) (status 20))
 (segment (start 137.16 142.367) (end 127 142.367) (width 1.905) (layer B.Cu) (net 6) (status 10))
 (segment (start 125.73 141.097) (end 124.527919 141.097) (width 1.905) (layer B.Cu) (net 6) (status 10))
 (segment (start 98.8695 114.2365) (end 98.8695 139.827) (width 1.905) (layer B.Cu) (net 6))
 (segment (start 98.8695 139.827) (end 98.933 139.827) (width 1.905) (layer B.Cu) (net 6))
 (segment (start 98.933 139.827) (end 106.934 147.828) (width 1.905) (layer B.Cu) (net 6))
 (segment (start 106.934 147.828) (end 107.696 147.828) (width 1.905) (layer B.Cu) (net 6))
 (segment (start 116.332 141.097) (end 115.1255 139.8905) (width 1.905) (layer B.Cu) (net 6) (status 20))
 (segment (start 125.73 141.097) (end 116.332 141.097) (width 1.905) (layer B.Cu) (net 6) (status 10))
 (segment (start 106.934 147.828) (end 107.6325 147.828) (width 1.905) (layer B.Cu) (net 6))
 (segment (start 107.6325 147.3835) (end 115.1255 139.8905) (width 1.905) (layer B.Cu) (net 6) (status 20))
 (segment (start 107.6325 147.828) (end 107.6325 147.3835) (width 1.905) (layer B.Cu) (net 6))
 (via (at 90.2335 113.8555) (size 1.778) (drill 0.889) (layers F.Cu B.Cu) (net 6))
 (segment (start 90.2335 108.208419) (end 90.2335 113.8555) (width 1.905) (layer B.Cu) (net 6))
 (segment (start 82.423 101.6) (end 83.625081 101.6) (width 1.905) (layer B.Cu) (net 6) (status 10))
 (segment (start 83.625081 101.6) (end 90.2335 108.208419) (width 1.905) (layer B.Cu) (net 6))
 (segment (start 126.38 122.667) (end 125.73 123.317) (width 1.905) (layer B.Cu) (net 8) (status 30))
 (segment (start 137.16 122.667) (end 126.38 122.667) (width 1.905) (layer B.Cu) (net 8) (status 30))
 (segment (start 102.743 124.46) (end 121.6025 124.46) (width 1.905) (layer B.Cu) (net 8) (status 10))
 (segment (start 122.7455 123.317) (end 125.73 123.317) (width 1.905) (layer B.Cu) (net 8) (status 20))
 (segment (start 121.6025 124.46) (end 122.7455 123.317) (width 1.905) (layer B.Cu) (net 8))
 (segment (start 130.048 113.157) (end 130.175 113.03) (width 1.905) (layer B.Cu) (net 5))
 (segment (start 130.048 113.792) (end 130.048 113.157) (width 1.905) (layer B.Cu) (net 5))
 (segment (start 110.236 113.792) (end 130.048 113.792) (width 1.905) (layer B.Cu) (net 5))
 (segment (start 83.82 91.948) (end 85.852 93.98) (width 1.905) (layer B.Cu) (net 5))
 (segment (start 80.264 91.948) (end 83.82 91.948) (width 1.905) (layer B.Cu) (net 5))
 (segment (start 88.9 103.124) (end 89.916 103.124) (width 1.905) (layer B.Cu) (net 5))
 (segment (start 78.8035 93.4085) (end 80.264 91.948) (width 1.905) (layer B.Cu) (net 5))
 (segment (start 78.8035 107.442) (end 78.8035 93.4085) (width 1.905) (layer B.Cu) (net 5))
 (segment (start 80.5815 109.22) (end 78.8035 107.442) (width 1.905) (layer B.Cu) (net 5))
 (segment (start 89.916 103.124) (end 94.996 98.044) (width 1.905) (layer B.Cu) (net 5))
 (segment (start 98.044 89.408) (end 105.664 89.408) (width 1.905) (layer B.Cu) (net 5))
 (segment (start 82.423 109.22) (end 80.5815 109.22) (width 1.905) (layer B.Cu) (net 5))
 (segment (start 85.852 93.98) (end 85.852 100.076) (width 1.905) (layer B.Cu) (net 5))
 (segment (start 85.852 100.076) (end 88.9 103.124) (width 1.905) (layer B.Cu) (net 5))
 (segment (start 94.996 98.044) (end 94.996 92.456) (width 1.905) (layer B.Cu) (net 5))
 (segment (start 105.664 89.408) (end 109.22 92.964) (width 1.905) (layer B.Cu) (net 5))
 (segment (start 94.996 92.456) (end 98.044 89.408) (width 1.905) (layer B.Cu) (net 5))
 (segment (start 109.22 92.964) (end 109.22 112.776) (width 1.905) (layer B.Cu) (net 5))
 (segment (start 109.22 112.776) (end 110.236 113.792) (width 1.905) (layer B.Cu) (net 5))
 (segment (start 102.743 111.76) (end 99.8855 111.76) (width 1.905) (layer B.Cu) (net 11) (status 10))
 (segment (start 99.8855 111.76) (end 99.1235 110.998) (width 1.905) (layer B.Cu) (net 11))
 (via (at 99.06 107.188) (size 1.778) (drill 0.889) (layers F.Cu B.Cu) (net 11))
 (segment (start 99.1235 110.998) (end 99.1235 107.2515) (width 1.905) (layer B.Cu) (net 11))
 (segment (start 99.1235 107.2515) (end 99.06 107.188) (width 1.905) (layer B.Cu) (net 11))
 (segment (start 119.4435 116.84) (end 115.7605 116.84) (width 1.905) (layer B.Cu) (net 11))
 (via (at 99.06 96.012) (size 1.778) (drill 0.889) (layers F.Cu B.Cu) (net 11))
 (segment (start 98.044 93.98) (end 98.044 94.996) (width 1.905) (layer B.Cu) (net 11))
 (segment (start 107.188 116.84) (end 106.172 115.824) (width 1.905) (layer B.Cu) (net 11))
 (segment (start 106.172 93.98) (end 104.14 91.948) (width 1.905) (layer B.Cu) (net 11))
 (segment (start 100.076 91.948) (end 98.044 93.98) (width 1.905) (layer B.Cu) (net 11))
 (segment (start 115.7605 116.84) (end 107.188 116.84) (width 1.905) (layer B.Cu) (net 11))
 (segment (start 104.14 91.948) (end 100.076 91.948) (width 1.905) (layer B.Cu) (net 11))
 (segment (start 98.044 94.996) (end 99.06 96.012) (width 1.905) (layer B.Cu) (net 11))
 (segment (start 106.172 115.824) (end 106.172 93.98) (width 1.905) (layer B.Cu) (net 11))
 (segment (start 82.423 119.38) (end 84.2645 119.38) (width 1.905) (layer B.Cu) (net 4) (status 10))
 (via (at 86.5505 108.585) (size 1.778) (drill 0.889) (layers F.Cu B.Cu) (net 4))
 (segment (start 84.2645 119.38) (end 86.5505 117.094) (width 1.905) (layer B.Cu) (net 4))
 (segment (start 86.5505 117.094) (end 86.5505 108.585) (width 1.905) (layer B.Cu) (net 4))
 (segment (start 130.175 110.49) (end 122.682 110.49) (width 1.905) (layer B.Cu) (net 4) (status 10))
 (segment (start 122.682 110.49) (end 115.062 110.49) (width 1.905) (layer B.Cu) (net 4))
 (segment (start 115.062 110.49) (end 114.046 110.49) (width 1.905) (layer B.Cu) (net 4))
 (segment (start 114.046 110.49) (end 112.268 108.712) (width 1.905) (layer B.Cu) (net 4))
 (segment (start 112.268 108.712) (end 112.268 90.932) (width 1.905) (layer B.Cu) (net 4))
 (segment (start 112.268 90.932) (end 107.696 86.36) (width 1.905) (layer B.Cu) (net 4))
 (segment (start 107.696 86.36) (end 96.012 86.36) (width 1.905) (layer B.Cu) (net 4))
 (segment (start 96.012 86.36) (end 95.504 86.36) (width 1.905) (layer B.Cu) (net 4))
 (segment (start 95.504 86.36) (end 89.408 92.456) (width 1.905) (layer B.Cu) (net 4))
 (via (at 89.408 99.568) (size 1.778) (drill 0.889) (layers F.Cu B.Cu) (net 4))
 (segment (start 89.408 92.456) (end 89.408 99.568) (width 1.905) (layer B.Cu) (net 4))
 (via (at 91.821 149.9235) (size 1.778) (drill 0.889) (layers F.Cu B.Cu) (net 9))
 (via (at 98.4885 143.764) (size 1.778) (drill 0.889) (layers F.Cu B.Cu) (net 9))
 (segment (start 102.5525 147.8915) (end 99.187 144.526) (width 1.905) (layer B.Cu) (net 9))
 (segment (start 99.187 144.4625) (end 98.4885 143.764) (width 1.905) (layer B.Cu) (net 9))
 (segment (start 99.187 144.526) (end 99.187 144.4625) (width 1.905) (layer B.Cu) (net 9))
 (segment (start 114.7835 145.7325) (end 114.7445 145.7715) (width 1.905) (layer B.Cu) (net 9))
 (segment (start 117.5385 145.7325) (end 114.7835 145.7325) (width 1.905) (layer B.Cu) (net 9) (status 10))
 (segment (start 114.7445 145.7715) (end 114.7445 147.447) (width 1.905) (layer B.Cu) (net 9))
 (segment (start 114.7445 147.447) (end 113.03 149.1615) (width 1.905) (layer B.Cu) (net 9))
 (segment (start 113.03 149.1615) (end 110.2995 149.1615) (width 1.905) (layer B.Cu) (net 9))
 (segment (start 110.2995 149.1615) (end 107.3785 152.0825) (width 1.905) (layer B.Cu) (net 9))
 (segment (start 107.3785 152.0825) (end 106.299 152.0825) (width 1.905) (layer B.Cu) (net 9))
 (segment (start 102.5525 148.336) (end 102.5525 147.8915) (width 1.905) (layer B.Cu) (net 9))
 (segment (start 106.299 152.0825) (end 102.5525 148.336) (width 1.905) (layer B.Cu) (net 9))
 (segment (start 89.789 139.3825) (end 89.789 147.8915) (width 1.905) (layer B.Cu) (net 9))
 (segment (start 78.9305 128.524) (end 89.789 139.3825) (width 1.905) (layer B.Cu) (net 9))
 (segment (start 78.9305 116.332) (end 78.9305 128.524) (width 1.905) (layer B.Cu) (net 9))
 (segment (start 89.789 147.8915) (end 91.821 149.9235) (width 1.905) (layer B.Cu) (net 9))
 (segment (start 82.423 114.3) (end 80.9625 114.3) (width 1.905) (layer B.Cu) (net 9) (status 10))
 (segment (start 80.9625 114.3) (end 78.9305 116.332) (width 1.905) (layer B.Cu) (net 9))
 (segment (start 79.4385 111.76) (end 82.423 111.76) (width 1.905) (layer B.Cu) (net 10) (status 20))
 (segment (start 78.486 112.7125) (end 79.4385 111.76) (width 1.905) (layer B.Cu) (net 10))
 (segment (start 78.486 112.7125) (end 78.486 112.776) (width 1.905) (layer B.Cu) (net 10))
 (segment (start 75.946 129.921) (end 75.946 115.316) (width 1.905) (layer B.Cu) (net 10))
 (segment (start 82.931 136.906) (end 75.946 129.921) (width 1.905) (layer B.Cu) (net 10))
 (segment (start 75.946 115.316) (end 76.0095 115.2525) (width 1.905) (layer B.Cu) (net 10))
 (segment (start 78.486 112.776) (end 76.0095 115.2525) (width 1.905) (layer B.Cu) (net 10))
 (segment (start 82.931 144.5895) (end 82.931 136.906) (width 1.905) (layer B.Cu) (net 10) (status 10))
 (segment (start 103.378 155.896919) (end 103.378 157.099) (width 1.905) (layer B.Cu) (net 12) (status 20))
 (segment (start 103.378 153.0985) (end 103.378 157.099) (width 1.905) (layer B.Cu) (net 12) (status 20))
 (segment (start 102.235 101.6) (end 102.1715 101.6635) (width 1.905) (layer B.Cu) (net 12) (status 30))
 (segment (start 102.743 101.6) (end 102.235 101.6) (width 1.905) (layer B.Cu) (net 12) (status 30))
 (segment (start 95.631 145.3515) (end 103.378 153.0985) (width 1.905) (layer B.Cu) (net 12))
 (segment (start 99.949 101.6635) (end 95.631 105.9815) (width 1.905) (layer B.Cu) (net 12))
 (segment (start 102.1715 101.6635) (end 99.949 101.6635) (width 1.905) (layer B.Cu) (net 12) (status 10))
 (segment (start 95.631 105.9815) (end 95.631 145.3515) (width 1.905) (layer B.Cu) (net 12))
 (segment (start 100.838 154.6225) (end 100.838 157.099) (width 1.905) (layer B.Cu) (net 13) (status 20))
 (segment (start 101.540919 99.06) (end 101.477419 98.9965) (width 1.905) (layer B.Cu) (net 13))
 (segment (start 102.743 99.06) (end 101.540919 99.06) (width 1.905) (layer B.Cu) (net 13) (status 10))
 (segment (start 101.477419 98.9965) (end 98.1075 98.9965) (width 1.905) (layer B.Cu) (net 13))
 (segment (start 98.1075 98.9965) (end 92.837 104.267) (width 1.905) (layer B.Cu) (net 13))
 (segment (start 92.837 104.267) (end 92.837 146.6215) (width 1.905) (layer B.Cu) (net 13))
 (segment (start 92.837 146.6215) (end 100.838 154.6225) (width 1.905) (layer B.Cu) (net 13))
 (segment (start 124.841 157.099) (end 126.453 157.099) (width 1.905) (layer B.Cu) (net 14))
 (segment (start 123.698 157.099) (end 124.841 157.099) (width 1.905) (layer B.Cu) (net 14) (status 10))
 (segment (start 120.1175 95.7825) (end 115.7605 100.1395) (width 1.905) (layer B.Cu) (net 14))
 (segment (start 135.4455 157.099) (end 149.1615 143.383) (width 1.905) (layer B.Cu) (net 14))
 (segment (start 144.5895 85.0265) (end 121.7295 85.0265) (width 1.905) (layer B.Cu) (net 14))
 (segment (start 124.841 157.099) (end 135.4455 157.099) (width 1.905) (layer B.Cu) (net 14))
 (segment (start 115.7605 90.9955) (end 115.7605 100.1395) (width 1.905) (layer B.Cu) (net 14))
 (segment (start 149.1615 143.383) (end 149.1615 89.5985) (width 1.905) (layer B.Cu) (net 14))
 (segment (start 149.1615 89.5985) (end 144.5895 85.0265) (width 1.905) (layer B.Cu) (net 14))
 (segment (start 121.7295 85.0265) (end 115.7605 90.9955) (width 1.905) (layer B.Cu) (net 14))
 (segment (start 120.777 95.123) (end 120.1175 95.7825) (width 1.905) (layer B.Cu) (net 14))
 (segment (start 122.8725 95.123) (end 120.777 95.123) (width 1.905) (layer B.Cu) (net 14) (status 10))
 (segment (start 115.7605 100.1395) (end 115.7605 106.68) (width 1.905) (layer B.Cu) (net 14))
 (segment (start 133.1595 91.948) (end 133.1595 93.433) (width 1.905) (layer B.Cu) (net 15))
 (segment (start 131.4695 95.123) (end 128.7145 95.123) (width 1.905) (layer B.Cu) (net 15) (status 20))
 (segment (start 133.1595 93.433) (end 131.4695 95.123) (width 1.905) (layer B.Cu) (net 15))
 (segment (start 141.947 91.948) (end 133.1595 91.948) (width 1.905) (layer B.Cu) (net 15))
 (segment (start 142.367 92.368) (end 141.947 91.948) (width 1.905) (layer B.Cu) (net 15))
 (segment (start 142.367 95.123) (end 142.367 92.368) (width 1.905) (layer B.Cu) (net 15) (status 10))
 (segment (start 139.827 96.325081) (end 133.155081 102.997) (width 1.905) (layer B.Cu) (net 3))
 (segment (start 139.827 95.123) (end 139.827 96.325081) (width 1.905) (layer B.Cu) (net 3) (status 10))
 (segment (start 133.028081 102.87) (end 130.175 102.87) (width 1.905) (layer B.Cu) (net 3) (status 20))
 (segment (start 133.155081 102.997) (end 133.028081 102.87) (width 1.905) (layer B.Cu) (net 3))
 (segment (start 116.688501 151.662499) (end 111.926001 151.662499) (width 1.905) (layer B.Cu) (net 16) (status 10))
 (segment (start 117.5385 150.8125) (end 116.688501 151.662499) (width 1.905) (layer B.Cu) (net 16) (status 30))
 (segment (start 108.458 155.1305) (end 108.458 157.099) (width 1.905) (layer B.Cu) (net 16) (status 20))
 (segment (start 111.926001 151.662499) (end 108.458 155.1305) (width 1.905) (layer B.Cu) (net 16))
 (segment (start 110.998 158.301081) (end 108.517081 160.782) (width 1.905) (layer B.Cu) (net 17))
 (segment (start 110.998 157.099) (end 110.998 158.301081) (width 1.905) (layer B.Cu) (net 17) (status 10))
 (segment (start 108.517081 160.782) (end 94.234 160.782) (width 1.905) (layer B.Cu) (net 17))
 (segment (start 94.234 160.782) (end 89.4715 156.0195) (width 1.905) (layer B.Cu) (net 17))
 (segment (start 89.4715 156.0195) (end 89.4715 152.0825) (width 1.905) (layer B.Cu) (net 17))
 (segment (start 89.4715 152.0825) (end 85.5345 148.1455) (width 1.905) (layer B.Cu) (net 17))
 (segment (start 85.471 146.3675) (end 85.471 144.5895) (width 1.905) (layer B.Cu) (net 17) (status 20))
 (segment (start 85.5345 146.431) (end 85.471 146.3675) (width 1.905) (layer B.Cu) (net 17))
 (segment (start 85.5345 146.431) (end 85.5345 144.5895) (width 1.905) (layer B.Cu) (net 17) (status 20))
 (segment (start 85.5345 148.1455) (end 85.5345 146.431) (width 1.905) (layer B.Cu) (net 17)))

